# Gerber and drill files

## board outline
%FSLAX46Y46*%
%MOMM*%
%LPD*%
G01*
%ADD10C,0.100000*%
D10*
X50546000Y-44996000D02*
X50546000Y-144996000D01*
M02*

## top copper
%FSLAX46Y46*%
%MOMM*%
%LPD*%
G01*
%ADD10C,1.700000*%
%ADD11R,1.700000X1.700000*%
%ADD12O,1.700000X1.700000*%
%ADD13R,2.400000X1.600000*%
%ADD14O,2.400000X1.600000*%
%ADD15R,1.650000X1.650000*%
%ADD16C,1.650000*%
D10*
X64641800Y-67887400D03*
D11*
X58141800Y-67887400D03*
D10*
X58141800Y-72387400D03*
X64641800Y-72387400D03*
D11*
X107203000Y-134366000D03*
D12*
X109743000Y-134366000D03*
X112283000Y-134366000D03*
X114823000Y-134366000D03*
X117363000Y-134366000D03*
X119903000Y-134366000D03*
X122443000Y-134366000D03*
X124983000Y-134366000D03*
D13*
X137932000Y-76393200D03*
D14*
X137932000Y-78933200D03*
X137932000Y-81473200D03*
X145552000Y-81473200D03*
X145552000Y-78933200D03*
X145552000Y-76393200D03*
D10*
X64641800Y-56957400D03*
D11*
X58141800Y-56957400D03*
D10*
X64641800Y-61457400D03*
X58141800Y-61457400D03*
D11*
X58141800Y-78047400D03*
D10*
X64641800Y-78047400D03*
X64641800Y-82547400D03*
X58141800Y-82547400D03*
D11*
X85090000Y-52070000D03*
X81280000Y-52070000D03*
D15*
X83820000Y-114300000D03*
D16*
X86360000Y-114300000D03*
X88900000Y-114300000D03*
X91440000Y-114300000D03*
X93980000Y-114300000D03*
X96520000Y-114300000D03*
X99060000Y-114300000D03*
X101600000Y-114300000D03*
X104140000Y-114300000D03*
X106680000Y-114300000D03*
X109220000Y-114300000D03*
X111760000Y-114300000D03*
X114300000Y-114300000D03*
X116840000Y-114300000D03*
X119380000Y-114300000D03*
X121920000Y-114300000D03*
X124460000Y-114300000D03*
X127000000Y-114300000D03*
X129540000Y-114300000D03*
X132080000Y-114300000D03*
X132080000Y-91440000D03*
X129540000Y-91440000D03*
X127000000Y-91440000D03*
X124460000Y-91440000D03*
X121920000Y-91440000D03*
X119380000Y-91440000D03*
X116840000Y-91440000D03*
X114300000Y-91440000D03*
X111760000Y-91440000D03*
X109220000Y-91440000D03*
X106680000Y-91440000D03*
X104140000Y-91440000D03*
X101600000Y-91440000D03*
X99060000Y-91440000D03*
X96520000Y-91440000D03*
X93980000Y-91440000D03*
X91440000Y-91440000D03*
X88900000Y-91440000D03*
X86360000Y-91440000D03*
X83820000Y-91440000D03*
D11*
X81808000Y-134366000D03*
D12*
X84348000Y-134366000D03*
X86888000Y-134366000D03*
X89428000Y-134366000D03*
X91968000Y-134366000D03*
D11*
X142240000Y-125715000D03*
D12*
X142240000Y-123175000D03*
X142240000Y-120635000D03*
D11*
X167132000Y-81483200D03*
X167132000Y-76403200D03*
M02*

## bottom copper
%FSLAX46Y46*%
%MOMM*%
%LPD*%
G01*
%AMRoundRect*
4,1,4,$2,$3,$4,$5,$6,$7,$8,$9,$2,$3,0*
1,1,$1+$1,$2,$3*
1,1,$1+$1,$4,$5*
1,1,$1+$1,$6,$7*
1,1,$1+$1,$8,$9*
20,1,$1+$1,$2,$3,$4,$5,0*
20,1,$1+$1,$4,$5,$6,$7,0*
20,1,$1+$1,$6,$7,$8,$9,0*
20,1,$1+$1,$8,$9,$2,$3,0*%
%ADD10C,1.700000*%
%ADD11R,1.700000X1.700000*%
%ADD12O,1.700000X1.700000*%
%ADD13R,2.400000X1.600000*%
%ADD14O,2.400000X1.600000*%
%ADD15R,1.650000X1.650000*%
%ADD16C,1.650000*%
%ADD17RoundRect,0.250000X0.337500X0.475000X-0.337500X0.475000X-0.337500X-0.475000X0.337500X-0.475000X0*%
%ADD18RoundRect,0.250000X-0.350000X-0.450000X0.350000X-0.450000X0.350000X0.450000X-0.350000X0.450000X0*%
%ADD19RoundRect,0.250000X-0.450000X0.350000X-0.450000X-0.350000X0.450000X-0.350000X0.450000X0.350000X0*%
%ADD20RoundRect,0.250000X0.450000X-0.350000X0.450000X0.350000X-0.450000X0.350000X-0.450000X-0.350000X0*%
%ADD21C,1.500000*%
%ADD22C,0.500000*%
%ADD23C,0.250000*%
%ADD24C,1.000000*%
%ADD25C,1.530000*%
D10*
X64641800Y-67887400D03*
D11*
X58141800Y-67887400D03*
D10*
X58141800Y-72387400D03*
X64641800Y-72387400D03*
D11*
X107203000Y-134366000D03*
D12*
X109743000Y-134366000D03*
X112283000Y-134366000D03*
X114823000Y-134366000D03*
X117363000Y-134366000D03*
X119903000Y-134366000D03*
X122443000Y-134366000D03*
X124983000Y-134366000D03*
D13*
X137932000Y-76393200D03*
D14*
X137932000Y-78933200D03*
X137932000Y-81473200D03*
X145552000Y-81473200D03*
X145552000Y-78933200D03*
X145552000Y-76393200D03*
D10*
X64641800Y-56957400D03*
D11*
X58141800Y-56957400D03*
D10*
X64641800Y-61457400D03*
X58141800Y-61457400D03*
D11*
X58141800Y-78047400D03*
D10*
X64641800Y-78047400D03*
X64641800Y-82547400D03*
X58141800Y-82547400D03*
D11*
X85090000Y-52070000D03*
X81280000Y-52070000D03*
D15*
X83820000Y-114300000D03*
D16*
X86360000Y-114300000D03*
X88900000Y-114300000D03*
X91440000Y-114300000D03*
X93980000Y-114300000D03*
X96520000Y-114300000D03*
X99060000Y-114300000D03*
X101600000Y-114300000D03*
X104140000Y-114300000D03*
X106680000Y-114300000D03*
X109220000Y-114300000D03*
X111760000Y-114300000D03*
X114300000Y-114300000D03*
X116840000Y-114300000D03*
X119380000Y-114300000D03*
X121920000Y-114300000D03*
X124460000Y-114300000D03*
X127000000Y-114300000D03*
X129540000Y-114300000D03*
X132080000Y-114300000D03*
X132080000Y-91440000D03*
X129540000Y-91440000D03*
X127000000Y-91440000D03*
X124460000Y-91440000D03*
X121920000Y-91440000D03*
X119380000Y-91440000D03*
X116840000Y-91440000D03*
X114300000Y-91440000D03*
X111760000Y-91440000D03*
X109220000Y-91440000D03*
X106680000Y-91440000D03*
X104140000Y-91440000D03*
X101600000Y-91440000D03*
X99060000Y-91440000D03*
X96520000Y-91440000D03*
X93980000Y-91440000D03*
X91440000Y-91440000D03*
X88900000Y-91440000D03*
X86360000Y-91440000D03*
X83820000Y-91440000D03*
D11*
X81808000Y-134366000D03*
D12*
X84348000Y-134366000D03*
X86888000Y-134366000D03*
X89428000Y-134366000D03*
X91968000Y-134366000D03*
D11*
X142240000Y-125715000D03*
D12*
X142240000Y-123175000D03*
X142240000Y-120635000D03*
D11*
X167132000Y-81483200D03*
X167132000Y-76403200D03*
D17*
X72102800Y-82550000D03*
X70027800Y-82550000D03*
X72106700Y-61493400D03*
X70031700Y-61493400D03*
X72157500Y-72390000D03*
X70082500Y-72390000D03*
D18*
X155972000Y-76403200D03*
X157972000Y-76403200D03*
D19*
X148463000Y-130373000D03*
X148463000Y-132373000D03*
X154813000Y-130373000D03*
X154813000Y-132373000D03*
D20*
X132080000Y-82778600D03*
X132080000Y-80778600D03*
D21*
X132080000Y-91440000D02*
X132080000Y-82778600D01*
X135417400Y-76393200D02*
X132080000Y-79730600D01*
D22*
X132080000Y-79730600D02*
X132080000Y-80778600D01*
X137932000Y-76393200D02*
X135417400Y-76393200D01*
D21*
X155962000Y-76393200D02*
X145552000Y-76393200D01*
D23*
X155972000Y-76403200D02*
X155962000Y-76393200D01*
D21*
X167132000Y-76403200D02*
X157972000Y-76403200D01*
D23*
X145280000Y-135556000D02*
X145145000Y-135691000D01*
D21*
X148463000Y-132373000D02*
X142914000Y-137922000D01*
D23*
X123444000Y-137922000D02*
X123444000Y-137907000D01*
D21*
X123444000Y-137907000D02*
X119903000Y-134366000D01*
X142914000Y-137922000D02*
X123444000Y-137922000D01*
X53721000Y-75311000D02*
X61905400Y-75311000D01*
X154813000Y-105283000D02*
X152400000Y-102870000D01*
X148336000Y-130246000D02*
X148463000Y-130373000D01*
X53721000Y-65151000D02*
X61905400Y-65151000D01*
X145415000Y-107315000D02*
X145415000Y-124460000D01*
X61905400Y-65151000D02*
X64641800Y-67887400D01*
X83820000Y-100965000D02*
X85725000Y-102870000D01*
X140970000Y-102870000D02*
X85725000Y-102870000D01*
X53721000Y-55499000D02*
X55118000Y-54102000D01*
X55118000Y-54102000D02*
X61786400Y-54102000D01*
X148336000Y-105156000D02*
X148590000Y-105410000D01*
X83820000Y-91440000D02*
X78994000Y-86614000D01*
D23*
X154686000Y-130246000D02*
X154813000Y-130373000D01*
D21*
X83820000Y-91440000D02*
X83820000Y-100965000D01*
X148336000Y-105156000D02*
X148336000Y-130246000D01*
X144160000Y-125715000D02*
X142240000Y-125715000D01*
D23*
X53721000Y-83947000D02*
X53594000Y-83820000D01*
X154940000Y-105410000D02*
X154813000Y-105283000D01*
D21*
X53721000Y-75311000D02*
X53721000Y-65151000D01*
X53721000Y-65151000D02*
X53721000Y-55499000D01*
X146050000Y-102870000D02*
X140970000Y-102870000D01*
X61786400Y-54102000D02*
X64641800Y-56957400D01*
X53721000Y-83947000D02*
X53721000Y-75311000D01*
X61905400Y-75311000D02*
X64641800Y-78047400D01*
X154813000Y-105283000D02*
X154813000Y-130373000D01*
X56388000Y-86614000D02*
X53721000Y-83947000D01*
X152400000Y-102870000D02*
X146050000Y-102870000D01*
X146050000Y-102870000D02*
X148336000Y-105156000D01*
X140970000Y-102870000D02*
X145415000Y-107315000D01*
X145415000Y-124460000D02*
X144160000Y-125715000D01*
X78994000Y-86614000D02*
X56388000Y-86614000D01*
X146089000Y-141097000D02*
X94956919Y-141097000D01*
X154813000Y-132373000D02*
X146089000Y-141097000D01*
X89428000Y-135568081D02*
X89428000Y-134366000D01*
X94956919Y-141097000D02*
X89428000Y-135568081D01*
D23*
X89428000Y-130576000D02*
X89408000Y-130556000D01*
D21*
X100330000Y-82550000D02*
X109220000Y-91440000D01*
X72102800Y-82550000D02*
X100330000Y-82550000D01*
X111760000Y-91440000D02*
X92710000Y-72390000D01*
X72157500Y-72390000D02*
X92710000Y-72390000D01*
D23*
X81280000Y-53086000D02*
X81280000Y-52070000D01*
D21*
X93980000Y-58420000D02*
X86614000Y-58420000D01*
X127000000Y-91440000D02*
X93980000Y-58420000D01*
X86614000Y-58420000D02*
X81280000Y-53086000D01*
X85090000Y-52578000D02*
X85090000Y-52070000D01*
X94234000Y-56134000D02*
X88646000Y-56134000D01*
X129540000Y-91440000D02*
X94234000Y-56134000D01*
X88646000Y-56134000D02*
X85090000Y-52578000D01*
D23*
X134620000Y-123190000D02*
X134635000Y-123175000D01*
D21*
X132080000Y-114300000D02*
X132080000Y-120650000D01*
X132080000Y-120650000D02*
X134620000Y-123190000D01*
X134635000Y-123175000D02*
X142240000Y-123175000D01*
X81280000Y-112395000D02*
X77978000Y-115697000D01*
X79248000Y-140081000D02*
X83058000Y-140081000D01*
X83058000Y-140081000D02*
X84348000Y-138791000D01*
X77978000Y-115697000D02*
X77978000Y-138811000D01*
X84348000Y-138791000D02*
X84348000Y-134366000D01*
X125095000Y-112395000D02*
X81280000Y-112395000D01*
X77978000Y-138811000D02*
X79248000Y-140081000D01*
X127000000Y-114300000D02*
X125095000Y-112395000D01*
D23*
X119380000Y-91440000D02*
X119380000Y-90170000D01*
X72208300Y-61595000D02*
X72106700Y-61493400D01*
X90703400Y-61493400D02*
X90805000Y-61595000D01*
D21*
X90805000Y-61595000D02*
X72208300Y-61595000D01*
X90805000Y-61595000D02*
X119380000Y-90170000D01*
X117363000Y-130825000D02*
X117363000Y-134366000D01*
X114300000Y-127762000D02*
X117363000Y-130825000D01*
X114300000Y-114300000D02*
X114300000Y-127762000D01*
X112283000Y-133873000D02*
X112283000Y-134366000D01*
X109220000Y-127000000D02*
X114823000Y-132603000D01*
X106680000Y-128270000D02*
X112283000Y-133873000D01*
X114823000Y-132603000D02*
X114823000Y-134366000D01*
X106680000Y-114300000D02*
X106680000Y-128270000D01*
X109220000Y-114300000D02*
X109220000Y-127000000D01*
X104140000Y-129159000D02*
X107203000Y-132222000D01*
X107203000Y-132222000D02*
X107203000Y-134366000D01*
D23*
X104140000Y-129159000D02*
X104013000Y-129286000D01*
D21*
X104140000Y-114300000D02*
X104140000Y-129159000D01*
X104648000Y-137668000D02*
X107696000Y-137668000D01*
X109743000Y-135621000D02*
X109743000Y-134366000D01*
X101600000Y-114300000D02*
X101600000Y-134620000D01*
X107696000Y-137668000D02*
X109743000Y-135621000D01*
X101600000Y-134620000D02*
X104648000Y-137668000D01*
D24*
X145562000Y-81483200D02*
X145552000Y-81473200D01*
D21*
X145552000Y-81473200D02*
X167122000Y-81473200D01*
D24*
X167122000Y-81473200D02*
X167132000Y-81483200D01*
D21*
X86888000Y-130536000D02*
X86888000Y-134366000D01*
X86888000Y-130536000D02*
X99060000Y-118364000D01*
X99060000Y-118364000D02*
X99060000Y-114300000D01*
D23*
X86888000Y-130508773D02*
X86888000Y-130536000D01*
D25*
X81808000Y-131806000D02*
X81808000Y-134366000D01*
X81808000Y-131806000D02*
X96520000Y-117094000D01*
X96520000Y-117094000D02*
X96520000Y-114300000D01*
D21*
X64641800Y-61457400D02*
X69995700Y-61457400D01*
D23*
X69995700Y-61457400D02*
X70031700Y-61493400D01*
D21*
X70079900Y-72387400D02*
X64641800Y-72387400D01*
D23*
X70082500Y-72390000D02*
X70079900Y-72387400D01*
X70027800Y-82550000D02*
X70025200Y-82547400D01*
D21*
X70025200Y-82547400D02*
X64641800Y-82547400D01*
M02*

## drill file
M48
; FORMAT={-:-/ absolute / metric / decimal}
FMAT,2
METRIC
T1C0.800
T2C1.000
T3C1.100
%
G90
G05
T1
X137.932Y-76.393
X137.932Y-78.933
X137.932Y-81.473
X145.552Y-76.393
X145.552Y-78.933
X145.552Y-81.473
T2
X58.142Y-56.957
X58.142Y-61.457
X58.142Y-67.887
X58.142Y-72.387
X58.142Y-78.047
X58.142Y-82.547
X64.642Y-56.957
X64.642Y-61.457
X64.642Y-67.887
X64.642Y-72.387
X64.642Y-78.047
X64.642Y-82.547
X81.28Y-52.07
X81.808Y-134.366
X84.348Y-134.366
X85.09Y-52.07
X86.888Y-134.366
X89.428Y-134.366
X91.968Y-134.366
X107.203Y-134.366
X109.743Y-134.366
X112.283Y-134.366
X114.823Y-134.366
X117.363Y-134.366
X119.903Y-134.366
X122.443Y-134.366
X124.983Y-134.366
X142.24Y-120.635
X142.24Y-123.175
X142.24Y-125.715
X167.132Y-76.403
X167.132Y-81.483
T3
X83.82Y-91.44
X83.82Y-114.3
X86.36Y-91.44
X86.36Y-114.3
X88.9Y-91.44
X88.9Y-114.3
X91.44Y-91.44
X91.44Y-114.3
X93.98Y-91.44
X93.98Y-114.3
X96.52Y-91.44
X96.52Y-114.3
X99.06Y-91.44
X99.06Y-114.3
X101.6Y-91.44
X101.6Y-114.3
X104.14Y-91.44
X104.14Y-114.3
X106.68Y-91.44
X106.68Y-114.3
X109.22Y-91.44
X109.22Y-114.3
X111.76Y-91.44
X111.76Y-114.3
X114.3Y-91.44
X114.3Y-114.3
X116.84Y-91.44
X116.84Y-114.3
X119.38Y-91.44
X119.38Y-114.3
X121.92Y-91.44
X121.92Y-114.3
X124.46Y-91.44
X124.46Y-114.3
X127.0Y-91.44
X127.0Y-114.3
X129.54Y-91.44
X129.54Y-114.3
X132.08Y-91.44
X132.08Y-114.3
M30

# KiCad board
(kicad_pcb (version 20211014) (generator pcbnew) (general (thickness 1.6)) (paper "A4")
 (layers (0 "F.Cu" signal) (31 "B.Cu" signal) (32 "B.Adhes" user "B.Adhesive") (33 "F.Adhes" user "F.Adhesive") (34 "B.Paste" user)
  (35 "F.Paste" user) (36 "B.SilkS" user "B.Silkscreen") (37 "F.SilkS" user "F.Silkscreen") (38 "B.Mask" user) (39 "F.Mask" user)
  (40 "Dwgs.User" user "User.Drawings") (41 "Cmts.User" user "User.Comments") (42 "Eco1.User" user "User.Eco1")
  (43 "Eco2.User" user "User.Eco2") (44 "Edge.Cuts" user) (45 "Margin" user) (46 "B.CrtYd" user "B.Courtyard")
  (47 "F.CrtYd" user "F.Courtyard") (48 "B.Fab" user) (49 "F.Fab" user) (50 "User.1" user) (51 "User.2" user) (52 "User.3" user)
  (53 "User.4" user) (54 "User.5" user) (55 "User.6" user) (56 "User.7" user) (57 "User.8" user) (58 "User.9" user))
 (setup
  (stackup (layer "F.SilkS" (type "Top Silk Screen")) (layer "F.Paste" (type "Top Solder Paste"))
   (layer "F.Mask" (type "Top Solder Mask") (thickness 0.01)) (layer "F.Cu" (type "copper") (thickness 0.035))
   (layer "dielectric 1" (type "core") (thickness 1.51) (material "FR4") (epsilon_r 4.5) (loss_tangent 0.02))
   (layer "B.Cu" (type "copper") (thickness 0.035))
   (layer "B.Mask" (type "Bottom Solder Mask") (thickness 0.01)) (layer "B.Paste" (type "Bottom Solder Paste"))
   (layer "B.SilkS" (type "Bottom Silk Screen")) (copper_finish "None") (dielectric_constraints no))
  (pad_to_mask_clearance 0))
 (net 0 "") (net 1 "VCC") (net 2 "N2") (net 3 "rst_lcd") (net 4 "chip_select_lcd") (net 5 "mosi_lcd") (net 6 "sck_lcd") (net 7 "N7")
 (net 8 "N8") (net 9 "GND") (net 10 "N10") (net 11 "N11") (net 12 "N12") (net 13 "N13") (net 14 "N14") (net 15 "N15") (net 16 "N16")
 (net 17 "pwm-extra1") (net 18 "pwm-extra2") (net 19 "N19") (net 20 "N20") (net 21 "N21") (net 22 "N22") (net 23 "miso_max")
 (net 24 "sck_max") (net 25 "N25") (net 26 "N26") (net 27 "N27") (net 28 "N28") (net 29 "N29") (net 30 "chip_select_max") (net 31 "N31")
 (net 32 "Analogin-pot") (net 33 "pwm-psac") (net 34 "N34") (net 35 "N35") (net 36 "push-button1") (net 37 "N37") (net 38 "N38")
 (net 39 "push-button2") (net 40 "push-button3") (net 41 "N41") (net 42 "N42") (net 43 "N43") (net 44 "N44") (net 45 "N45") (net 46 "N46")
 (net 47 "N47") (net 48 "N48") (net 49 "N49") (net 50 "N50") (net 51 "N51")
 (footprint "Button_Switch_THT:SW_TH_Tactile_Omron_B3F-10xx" (layer "F.Cu") (at 58.1418 67.8874)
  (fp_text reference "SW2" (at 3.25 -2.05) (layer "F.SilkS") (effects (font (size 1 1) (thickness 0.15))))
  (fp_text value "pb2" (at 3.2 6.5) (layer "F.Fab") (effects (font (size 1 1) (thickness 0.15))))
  (pad "1" thru_hole circle (at 6.5 0) (size 1.7 1.7) (drill 1) (layers *.Cu *.Mask) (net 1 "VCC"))
  (pad "1" thru_hole rect (at 0 0) (size 1.7 1.7) (drill 1) (layers *.Cu *.Mask) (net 1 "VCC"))
  (pad "2" thru_hole circle (at 0 4.5) (size 1.7 1.7) (drill 1) (layers *.Cu *.Mask) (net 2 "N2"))
  (pad "2" thru_hole circle (at 6.5 4.5) (size 1.7 1.7) (drill 1) (layers *.Cu *.Mask) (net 2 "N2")))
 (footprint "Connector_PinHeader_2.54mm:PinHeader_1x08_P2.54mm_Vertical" (layer "F.Cu") (at 107.203 134.366 90)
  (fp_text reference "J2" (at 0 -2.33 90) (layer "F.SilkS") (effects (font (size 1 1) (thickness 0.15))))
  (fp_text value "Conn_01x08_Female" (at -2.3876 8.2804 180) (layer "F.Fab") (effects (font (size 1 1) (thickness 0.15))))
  (pad "1" thru_hole rect (at 0 0 90) (size 1.7 1.7) (drill 1) (layers *.Cu *.Mask) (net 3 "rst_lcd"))
  (pad "2" thru_hole oval (at 0 2.54 90) (size 1.7 1.7) (drill 1) (layers *.Cu *.Mask) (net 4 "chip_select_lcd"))
  (pad "3" thru_hole oval (at 0 5.08 90) (size 1.7 1.7) (drill 1) (layers *.Cu *.Mask) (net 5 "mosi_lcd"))
  (pad "4" thru_hole oval (at 0 7.62 90) (size 1.7 1.7) (drill 1) (layers *.Cu *.Mask) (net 5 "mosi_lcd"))
  (pad "5" thru_hole oval (at 0 10.16 90) (size 1.7 1.7) (drill 1) (layers *.Cu *.Mask) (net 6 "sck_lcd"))
  (pad "6" thru_hole oval (at 0 12.7 90) (size 1.7 1.7) (drill 1) (layers *.Cu *.Mask) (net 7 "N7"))
  (pad "7" thru_hole oval (at 0 15.24 90) (size 1.7 1.7) (drill 1) (layers *.Cu *.Mask) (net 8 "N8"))
  (pad "8" thru_hole oval (at 0 17.78 90) (size 1.7 1.7) (drill 1) (layers *.Cu *.Mask) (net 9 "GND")))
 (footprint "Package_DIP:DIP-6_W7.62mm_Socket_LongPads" (layer "F.Cu") (at 137.932 76.3932)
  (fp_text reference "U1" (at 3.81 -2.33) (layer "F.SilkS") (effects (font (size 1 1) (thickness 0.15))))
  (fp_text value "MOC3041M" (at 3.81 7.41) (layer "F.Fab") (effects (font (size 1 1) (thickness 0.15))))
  (pad "1" thru_hole rect (at 0 0) (size 2.4 1.6) (drill 0.8) (layers *.Cu *.Mask) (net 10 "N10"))
  (pad "2" thru_hole oval (at 0 2.54) (size 2.4 1.6) (drill 0.8) (layers *.Cu *.Mask) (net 9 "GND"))
  (pad "3" thru_hole oval (at 0 5.08) (size 2.4 1.6) (drill 0.8) (layers *.Cu *.Mask) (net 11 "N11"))
  (pad "4" thru_hole oval (at 7.62 5.08) (size 2.4 1.6) (drill 0.8) (layers *.Cu *.Mask) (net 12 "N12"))
  (pad "5" thru_hole oval (at 7.62 2.54) (size 2.4 1.6) (drill 0.8) (layers *.Cu *.Mask) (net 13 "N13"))
  (pad "6" thru_hole oval (at 7.62 0) (size 2.4 1.6) (drill 0.8) (layers *.Cu *.Mask) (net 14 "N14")))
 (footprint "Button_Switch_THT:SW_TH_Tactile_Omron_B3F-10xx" (layer "F.Cu") (at 58.1418 56.9574)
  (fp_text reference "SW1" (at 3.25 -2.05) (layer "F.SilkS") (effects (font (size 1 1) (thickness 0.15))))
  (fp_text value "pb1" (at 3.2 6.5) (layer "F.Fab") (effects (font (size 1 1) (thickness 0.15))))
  (pad "1" thru_hole circle (at 6.5 0) (size 1.7 1.7) (drill 1) (layers *.Cu *.Mask) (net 1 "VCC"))
  (pad "1" thru_hole rect (at 0 0) (size 1.7 1.7) (drill 1) (layers *.Cu *.Mask) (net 1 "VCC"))
  (pad "2" thru_hole circle (at 6.5 4.5) (size 1.7 1.7) (drill 1) (layers *.Cu *.Mask) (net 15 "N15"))
  (pad "2" thru_hole circle (at 0 4.5) (size 1.7 1.7) (drill 1) (layers *.Cu *.Mask) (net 15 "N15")))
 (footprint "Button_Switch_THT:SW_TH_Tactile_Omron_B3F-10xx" (layer "F.Cu") (at 58.1418 78.0474)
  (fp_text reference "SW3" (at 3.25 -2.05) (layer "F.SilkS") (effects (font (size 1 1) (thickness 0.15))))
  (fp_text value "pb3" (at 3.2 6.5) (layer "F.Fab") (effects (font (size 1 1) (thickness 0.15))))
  (pad "1" thru_hole rect (at 0 0) (size 1.7 1.7) (drill 1) (layers *.Cu *.Mask) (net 1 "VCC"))
  (pad "1" thru_hole circle (at 6.5 0) (size 1.7 1.7) (drill 1) (layers *.Cu *.Mask) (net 1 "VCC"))
  (pad "2" thru_hole circle (at 6.5 4.5) (size 1.7 1.7) (drill 1) (layers *.Cu *.Mask) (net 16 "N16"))
  (pad "2" thru_hole circle (at 0 4.5) (size 1.7 1.7) (drill 1) (layers *.Cu *.Mask) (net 16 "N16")))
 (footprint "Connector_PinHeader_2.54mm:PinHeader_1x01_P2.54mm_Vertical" (layer "F.Cu") (at 85.09 52.07)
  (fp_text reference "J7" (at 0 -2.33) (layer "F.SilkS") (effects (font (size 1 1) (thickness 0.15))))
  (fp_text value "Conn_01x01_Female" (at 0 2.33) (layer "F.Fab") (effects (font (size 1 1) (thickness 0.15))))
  (pad "1" thru_hole rect (at 0 0) (size 1.7 1.7) (drill 1) (layers *.Cu *.Mask) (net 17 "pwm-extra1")))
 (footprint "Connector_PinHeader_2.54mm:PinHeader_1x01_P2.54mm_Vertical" (layer "F.Cu") (at 81.28 52.07)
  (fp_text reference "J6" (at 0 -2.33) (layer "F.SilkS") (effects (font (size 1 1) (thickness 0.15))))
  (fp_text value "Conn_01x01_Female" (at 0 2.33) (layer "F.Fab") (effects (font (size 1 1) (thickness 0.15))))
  (pad "1" thru_hole rect (at 0 0) (size 1.7 1.7) (drill 1) (layers *.Cu *.Mask) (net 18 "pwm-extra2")))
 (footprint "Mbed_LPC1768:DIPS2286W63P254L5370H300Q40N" (layer "F.Cu") (at 83.82 114.3 90)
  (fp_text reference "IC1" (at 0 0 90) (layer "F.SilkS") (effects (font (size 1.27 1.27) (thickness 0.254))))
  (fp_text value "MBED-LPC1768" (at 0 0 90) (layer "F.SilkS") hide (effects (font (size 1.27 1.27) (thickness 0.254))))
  (pad "1" thru_hole rect locked (at 0 0 90) (size 1.65 1.65) (drill 1.1) (layers *.Cu *.Mask) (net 9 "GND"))
  (pad "2" thru_hole circle locked (at 0 2.54 90) (size 1.65 1.65) (drill 1.1) (layers *.Cu *.Mask) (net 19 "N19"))
  (pad "3" thru_hole circle locked (at 0 5.08 90) (size 1.65 1.65) (drill 1.1) (layers *.Cu *.Mask) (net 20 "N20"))
  (pad "4" thru_hole circle locked (at 0 7.62 90) (size 1.65 1.65) (drill 1.1) (layers *.Cu *.Mask) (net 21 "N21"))
  (pad "5" thru_hole circle locked (at 0 10.16 90) (size 1.65 1.65) (drill 1.1) (layers *.Cu *.Mask) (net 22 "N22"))
  (pad "6" thru_hole circle locked (at 0 12.7 90) (size 1.65 1.65) (drill 1.1) (layers *.Cu *.Mask) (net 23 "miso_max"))
  (pad "7" thru_hole circle locked (at 0 15.24 90) (size 1.65 1.65) (drill 1.1) (layers *.Cu *.Mask) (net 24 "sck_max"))
  (pad "8" thru_hole circle locked (at 0 17.78 90) (size 1.65 1.65) (drill 1.1) (layers *.Cu *.Mask) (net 4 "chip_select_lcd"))
  (pad "9" thru_hole circle locked (at 0 20.32 90) (size 1.65 1.65) (drill 1.1) (layers *.Cu *.Mask) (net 3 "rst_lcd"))
  (pad "10" thru_hole circle locked (at 0 22.86 90) (size 1.65 1.65) (drill 1.1) (layers *.Cu *.Mask) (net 5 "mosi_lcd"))
  (pad "11" thru_hole circle locked (at 0 25.4 90) (size 1.65 1.65) (drill 1.1) (layers *.Cu *.Mask) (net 5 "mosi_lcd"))
  (pad "12" thru_hole circle locked (at 0 27.94 90) (size 1.65 1.65) (drill 1.1) (layers *.Cu *.Mask) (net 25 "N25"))
  (pad "13" thru_hole circle locked (at 0 30.48 90) (size 1.65 1.65) (drill 1.1) (layers *.Cu *.Mask) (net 6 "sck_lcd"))
  (pad "14" thru_hole circle locked (at 0 33.02 90) (size 1.65 1.65) (drill 1.1) (layers *.Cu *.Mask) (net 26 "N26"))
  (pad "15" thru_hole circle locked (at 0 35.56 90) (size 1.65 1.65) (drill 1.1) (layers *.Cu *.Mask) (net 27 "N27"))
  (pad "16" thru_hole circle locked (at 0 38.1 90) (size 1.65 1.65) (drill 1.1) (layers *.Cu *.Mask) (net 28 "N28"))
  (pad "17" thru_hole circle locked (at 0 40.64 90) (size 1.65 1.65) (drill 1.1) (layers *.Cu *.Mask) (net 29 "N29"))
  (pad "18" thru_hole circle locked (at 0 43.18 90) (size 1.65 1.65) (drill 1.1) (layers *.Cu *.Mask) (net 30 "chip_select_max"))
  (pad "19" thru_hole circle locked (at 0 45.72 90) (size 1.65 1.65) (drill 1.1) (layers *.Cu *.Mask) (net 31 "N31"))
  (pad "20" thru_hole circle locked (at 0 48.26 90) (size 1.65 1.65) (drill 1.1) (layers *.Cu *.Mask) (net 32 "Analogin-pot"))
  (pad "21" thru_hole circle locked (at 22.86 48.26 90) (size 1.65 1.65) (drill 1.1) (layers *.Cu *.Mask) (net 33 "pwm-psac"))
  (pad "22" thru_hole circle locked (at 22.86 45.72 90) (size 1.65 1.65) (drill 1.1) (layers *.Cu *.Mask) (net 17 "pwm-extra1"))
  (pad "23" thru_hole circle locked (at 22.86 43.18 90) (size 1.65 1.65) (drill 1.1) (layers *.Cu *.Mask) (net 18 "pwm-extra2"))
  (pad "24" thru_hole circle locked (at 22.86 40.64 90) (size 1.65 1.65) (drill 1.1) (layers *.Cu *.Mask) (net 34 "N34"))
  (pad "25" thru_hole circle locked (at 22.86 38.1 90) (size 1.65 1.65) (drill 1.1) (layers *.Cu *.Mask) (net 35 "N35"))
  (pad "26" thru_hole circle locked (at 22.86 35.56 90) (size 1.65 1.65) (drill 1.1) (layers *.Cu *.Mask) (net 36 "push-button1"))
  (pad "27" thru_hole circle locked (at 22.86 33.02 90) (size 1.65 1.65) (drill 1.1) (layers *.Cu *.Mask) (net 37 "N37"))
  (pad "28" thru_hole circle locked (at 22.86 30.48 90) (size 1.65 1.65) (drill 1.1) (layers *.Cu *.Mask) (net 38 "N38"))
  (pad "29" thru_hole circle locked (at 22.86 27.94 90) (size 1.65 1.65) (drill 1.1) (layers *.Cu *.Mask) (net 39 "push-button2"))
  (pad "30" thru_hole circle locked (at 22.86 25.4 90) (size 1.65 1.65) (drill 1.1) (layers *.Cu *.Mask) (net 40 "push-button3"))
  (pad "31" thru_hole circle locked (at 22.86 22.86 90) (size 1.65 1.65) (drill 1.1) (layers *.Cu *.Mask) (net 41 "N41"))
  (pad "32" thru_hole circle locked (at 22.86 20.32 90) (size 1.65 1.65) (drill 1.1) (layers *.Cu *.Mask) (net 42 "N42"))
  (pad "33" thru_hole circle locked (at 22.86 17.78 90) (size 1.65 1.65) (drill 1.1) (layers *.Cu *.Mask) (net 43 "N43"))
  (pad "34" thru_hole circle locked (at 22.86 15.24 90) (size 1.65 1.65) (drill 1.1) (layers *.Cu *.Mask) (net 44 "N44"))
  (pad "35" thru_hole circle locked (at 22.86 12.7 90) (size 1.65 1.65) (drill 1.1) (layers *.Cu *.Mask) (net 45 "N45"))
  (pad "36" thru_hole circle locked (at 22.86 10.16 90) (size 1.65 1.65) (drill 1.1) (layers *.Cu *.Mask) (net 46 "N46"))
  (pad "37" thru_hole circle locked (at 22.86 7.62 90) (size 1.65 1.65) (drill 1.1) (layers *.Cu *.Mask) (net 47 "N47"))
  (pad "38" thru_hole circle locked (at 22.86 5.08 90) (size 1.65 1.65) (drill 1.1) (layers *.Cu *.Mask) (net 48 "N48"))
  (pad "39" thru_hole circle locked (at 22.86 2.54 90) (size 1.65 1.65) (drill 1.1) (layers *.Cu *.Mask) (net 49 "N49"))
  (pad "40" thru_hole circle locked (at 22.86 0 90) (size 1.65 1.65) (drill 1.1) (layers *.Cu *.Mask) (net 1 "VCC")))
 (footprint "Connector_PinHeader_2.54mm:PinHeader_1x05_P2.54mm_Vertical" (layer "F.Cu") (at 81.808 134.366 90)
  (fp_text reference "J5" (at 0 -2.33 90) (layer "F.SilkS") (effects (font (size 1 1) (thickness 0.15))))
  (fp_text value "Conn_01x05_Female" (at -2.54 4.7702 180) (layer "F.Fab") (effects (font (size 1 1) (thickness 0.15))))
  (pad "1" thru_hole rect (at 0 0 90) (size 1.7 1.7) (drill 1) (layers *.Cu *.Mask) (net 23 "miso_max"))
  (pad "2" thru_hole oval (at 0 2.54 90) (size 1.7 1.7) (drill 1) (layers *.Cu *.Mask) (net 30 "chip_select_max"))
  (pad "3" thru_hole oval (at 0 5.08 90) (size 1.7 1.7) (drill 1) (layers *.Cu *.Mask) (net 24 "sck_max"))
  (pad "4" thru_hole oval (at 0 7.62 90) (size 1.7 1.7) (drill 1) (layers *.Cu *.Mask) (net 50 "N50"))
  (pad "5" thru_hole oval (at 0 10.16 90) (size 1.7 1.7) (drill 1) (layers *.Cu *.Mask) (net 9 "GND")))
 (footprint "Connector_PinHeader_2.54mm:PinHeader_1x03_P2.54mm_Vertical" (layer "F.Cu") (at 142.24 125.715 180)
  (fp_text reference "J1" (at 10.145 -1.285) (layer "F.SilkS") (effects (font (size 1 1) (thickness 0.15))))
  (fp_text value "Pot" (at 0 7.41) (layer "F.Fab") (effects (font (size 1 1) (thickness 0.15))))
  (pad "1" thru_hole rect (at 0 0 180) (size 1.7 1.7) (drill 1) (layers *.Cu *.Mask) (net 1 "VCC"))
  (pad "2" thru_hole oval (at 0 2.54 180) (size 1.7 1.7) (drill 1) (layers *.Cu *.Mask) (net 32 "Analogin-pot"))
  (pad "3" thru_hole oval (at 0 5.08 180) (size 1.7 1.7) (drill 1) (layers *.Cu *.Mask) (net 9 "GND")))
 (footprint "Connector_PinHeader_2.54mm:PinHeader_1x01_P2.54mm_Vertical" (layer "F.Cu") (at 167.132 81.4832)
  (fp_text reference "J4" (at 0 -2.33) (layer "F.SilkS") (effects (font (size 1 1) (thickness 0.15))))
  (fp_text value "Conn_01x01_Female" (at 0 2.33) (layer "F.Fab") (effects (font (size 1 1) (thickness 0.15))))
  (pad "1" thru_hole rect (at 0 0) (size 1.7 1.7) (drill 1) (layers *.Cu *.Mask) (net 12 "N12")))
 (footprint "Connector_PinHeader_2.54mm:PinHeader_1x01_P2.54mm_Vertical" (layer "F.Cu") (at 167.132 76.4032)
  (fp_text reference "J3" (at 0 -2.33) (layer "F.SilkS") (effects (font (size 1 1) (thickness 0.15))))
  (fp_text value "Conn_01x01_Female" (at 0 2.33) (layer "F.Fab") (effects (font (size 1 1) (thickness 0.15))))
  (pad "1" thru_hole rect (at 0 0) (size 1.7 1.7) (drill 1) (layers *.Cu *.Mask) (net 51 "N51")))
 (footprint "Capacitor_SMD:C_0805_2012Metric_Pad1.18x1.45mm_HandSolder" (layer "B.Cu") (at 71.0653 82.55 180)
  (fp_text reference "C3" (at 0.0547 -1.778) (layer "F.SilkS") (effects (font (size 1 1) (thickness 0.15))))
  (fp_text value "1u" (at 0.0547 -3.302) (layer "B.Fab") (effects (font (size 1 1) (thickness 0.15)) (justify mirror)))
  (pad "1" smd roundrect (at -1.0375 0 180) (size 1.175 1.45) (layers "B.Cu" "B.Paste" "B.Mask") (roundrect_rratio 0.212766)
   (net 40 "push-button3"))
  (pad "2" smd roundrect (at 1.0375 0 180) (size 1.175 1.45) (layers "B.Cu" "B.Paste" "B.Mask") (roundrect_rratio 0.212766) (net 16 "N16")))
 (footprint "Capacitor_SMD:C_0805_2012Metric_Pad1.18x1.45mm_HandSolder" (layer "B.Cu") (at 71.0692 61.4934 180)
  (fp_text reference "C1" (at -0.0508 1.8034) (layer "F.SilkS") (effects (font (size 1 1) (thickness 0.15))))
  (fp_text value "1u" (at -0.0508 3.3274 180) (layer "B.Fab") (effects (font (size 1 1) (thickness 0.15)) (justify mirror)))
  (pad "1" smd roundrect (at -1.0375 0 180) (size 1.175 1.45) (layers "B.Cu" "B.Paste" "B.Mask") (roundrect_rratio 0.212766)
   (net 36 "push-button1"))
  (pad "2" smd roundrect (at 1.0375 0 180) (size 1.175 1.45) (layers "B.Cu" "B.Paste" "B.Mask") (roundrect_rratio 0.212766) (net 15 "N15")))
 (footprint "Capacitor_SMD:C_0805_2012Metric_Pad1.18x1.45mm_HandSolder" (layer "B.Cu") (at 71.12 72.39 180)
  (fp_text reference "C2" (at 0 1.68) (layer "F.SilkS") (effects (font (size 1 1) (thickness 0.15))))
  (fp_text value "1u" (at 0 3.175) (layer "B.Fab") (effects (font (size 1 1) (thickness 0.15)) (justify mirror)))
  (pad "1" smd roundrect (at -1.0375 0 180) (size 1.175 1.45) (layers "B.Cu" "B.Paste" "B.Mask") (roundrect_rratio 0.212766)
   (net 39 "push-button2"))
  (pad "2" smd roundrect (at 1.0375 0 180) (size 1.175 1.45) (layers "B.Cu" "B.Paste" "B.Mask") (roundrect_rratio 0.212766) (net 2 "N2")))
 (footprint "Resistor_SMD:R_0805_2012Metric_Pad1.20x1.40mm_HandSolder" (layer "B.Cu") (at 156.972 76.4032)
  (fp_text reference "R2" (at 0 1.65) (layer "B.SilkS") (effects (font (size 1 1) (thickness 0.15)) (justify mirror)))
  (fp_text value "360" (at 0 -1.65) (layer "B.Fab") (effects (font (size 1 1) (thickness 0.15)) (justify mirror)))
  (pad "1" smd roundrect (at -1 0) (size 1.2 1.4) (layers "B.Cu" "B.Paste" "B.Mask") (roundrect_rratio 0.2083333333) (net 14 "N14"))
  (pad "2" smd roundrect (at 1 0) (size 1.2 1.4) (layers "B.Cu" "B.Paste" "B.Mask") (roundrect_rratio 0.2083333333) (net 51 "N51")))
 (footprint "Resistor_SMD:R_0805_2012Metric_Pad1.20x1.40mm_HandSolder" (layer "B.Cu") (at 148.463 131.373 -90)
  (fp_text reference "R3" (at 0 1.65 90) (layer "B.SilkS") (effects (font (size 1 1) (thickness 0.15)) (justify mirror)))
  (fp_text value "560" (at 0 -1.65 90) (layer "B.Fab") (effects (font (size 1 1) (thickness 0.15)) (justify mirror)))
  (pad "1" smd roundrect (at -1 0 270) (size 1.2 1.4) (layers "B.Cu" "B.Paste" "B.Mask") (roundrect_rratio 0.208333) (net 1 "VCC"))
  (pad "2" smd roundrect (at 1 0 270) (size 1.2 1.4) (layers "B.Cu" "B.Paste" "B.Mask") (roundrect_rratio 0.208333) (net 7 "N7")))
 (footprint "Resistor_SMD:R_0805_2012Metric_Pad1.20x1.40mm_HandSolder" (layer "B.Cu") (at 154.813 131.373 -90)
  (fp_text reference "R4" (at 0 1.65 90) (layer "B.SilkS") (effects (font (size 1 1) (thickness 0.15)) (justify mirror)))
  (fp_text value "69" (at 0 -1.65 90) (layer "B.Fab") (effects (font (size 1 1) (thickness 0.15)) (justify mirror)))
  (pad "1" smd roundrect (at -1 0 270) (size 1.2 1.4) (layers "B.Cu" "B.Paste" "B.Mask") (roundrect_rratio 0.208333) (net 1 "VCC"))
  (pad "2" smd roundrect (at 1 0 270) (size 1.2 1.4) (layers "B.Cu" "B.Paste" "B.Mask") (roundrect_rratio 0.208333) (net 50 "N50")))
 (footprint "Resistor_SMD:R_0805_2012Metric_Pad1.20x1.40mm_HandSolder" (layer "B.Cu") (at 132.08 81.7786 90)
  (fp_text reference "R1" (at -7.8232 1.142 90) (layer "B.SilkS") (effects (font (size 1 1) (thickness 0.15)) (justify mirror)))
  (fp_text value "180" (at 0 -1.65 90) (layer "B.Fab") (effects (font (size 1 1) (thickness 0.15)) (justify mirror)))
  (pad "1" smd roundrect (at -1 0 90) (size 1.2 1.4) (layers "B.Cu" "B.Paste" "B.Mask") (roundrect_rratio 0.2083333333) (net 33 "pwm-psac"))
  (pad "2" smd roundrect (at 1 0 90) (size 1.2 1.4) (layers "B.Cu" "B.Paste" "B.Mask") (roundrect_rratio 0.2083333333) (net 10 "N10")))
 (gr_line (start 50.546 44.996) (end 50.546 144.996) (layer "Edge.Cuts") (width 0.1))
 (segment (start 132.08 91.44) (end 132.08 82.7786) (width 1.5) (layer "B.Cu") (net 33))
 (segment (start 135.4174 76.3932) (end 132.08 79.7306) (width 1.5) (layer "B.Cu") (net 10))
 (segment (start 132.08 79.7306) (end 132.08 80.7786) (width 0.5) (layer "B.Cu") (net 10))
 (segment (start 137.932 76.3932) (end 135.4174 76.3932) (width 0.5) (layer "B.Cu") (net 10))
 (segment (start 155.962 76.3932) (end 145.552 76.3932) (width 1.5) (layer "B.Cu") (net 14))
 (segment (start 155.972 76.4032) (end 155.962 76.3932) (width 0.25) (layer "B.Cu") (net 14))
 (segment (start 167.132 76.4032) (end 157.972 76.4032) (width 1.5) (layer "B.Cu") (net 51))
 (segment (start 145.28 135.556) (end 145.145 135.691) (width 0.25) (layer "B.Cu") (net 7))
 (segment (start 148.463 132.373) (end 142.914 137.922) (width 1.5) (layer "B.Cu") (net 7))
 (segment (start 123.444 137.922) (end 123.444 137.907) (width 0.25) (layer "B.Cu") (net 7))
 (segment (start 123.444 137.907) (end 119.903 134.366) (width 1.5) (layer "B.Cu") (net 7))
 (segment (start 142.914 137.922) (end 123.444 137.922) (width 1.5) (layer "B.Cu") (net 7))
 (segment (start 53.721 75.311) (end 61.9054 75.311) (width 1.5) (layer "B.Cu") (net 1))
 (segment (start 154.813 105.283) (end 152.4 102.87) (width 1.5) (layer "B.Cu") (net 1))
 (segment (start 148.336 130.246) (end 148.463 130.373) (width 1.5) (layer "B.Cu") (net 1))
 (segment (start 53.721 65.151) (end 61.9054 65.151) (width 1.5) (layer "B.Cu") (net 1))
 (segment (start 145.415 107.315) (end 145.415 124.46) (width 1.5) (layer "B.Cu") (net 1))
 (segment (start 61.9054 65.151) (end 64.6418 67.8874) (width 1.5) (layer "B.Cu") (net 1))
 (segment (start 83.82 100.965) (end 85.725 102.87) (width 1.5) (layer "B.Cu") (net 1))
 (segment (start 140.97 102.87) (end 85.725 102.87) (width 1.5) (layer "B.Cu") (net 1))
 (segment (start 53.721 55.499) (end 55.118 54.102) (width 1.5) (layer "B.Cu") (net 1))
 (segment (start 55.118 54.102) (end 61.7864 54.102) (width 1.5) (layer "B.Cu") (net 1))
 (segment (start 148.336 105.156) (end 148.59 105.41) (width 1.5) (layer "B.Cu") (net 1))
 (segment (start 83.82 91.44) (end 78.994 86.614) (width 1.5) (layer "B.Cu") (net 1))
 (segment (start 154.686 130.246) (end 154.813 130.373) (width 0.25) (layer "B.Cu") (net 1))
 (segment (start 83.82 91.44) (end 83.82 100.965) (width 1.5) (layer "B.Cu") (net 1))
 (segment (start 148.336 105.156) (end 148.336 130.246) (width 1.5) (layer "B.Cu") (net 1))
 (segment (start 144.16 125.715) (end 142.24 125.715) (width 1.5) (layer "B.Cu") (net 1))
 (segment (start 53.721 83.947) (end 53.594 83.82) (width 0.25) (layer "B.Cu") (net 1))
 (segment (start 154.94 105.41) (end 154.813 105.283) (width 0.25) (layer "B.Cu") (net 1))
 (segment (start 53.721 75.311) (end 53.721 65.151) (width 1.5) (layer "B.Cu") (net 1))
 (segment (start 53.721 65.151) (end 53.721 55.499) (width 1.5) (layer "B.Cu") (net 1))
 (segment (start 146.05 102.87) (end 140.97 102.87) (width 1.5) (layer "B.Cu") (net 1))
 (segment (start 61.7864 54.102) (end 64.6418 56.9574) (width 1.5) (layer "B.Cu") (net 1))
 (segment (start 53.721 83.947) (end 53.721 75.311) (width 1.5) (layer "B.Cu") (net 1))
 (segment (start 61.9054 75.311) (end 64.6418 78.0474) (width 1.5) (layer "B.Cu") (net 1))
 (segment (start 154.813 105.283) (end 154.813 130.373) (width 1.5) (layer "B.Cu") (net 1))
 (segment (start 56.388 86.614) (end 53.721 83.947) (width 1.5) (layer "B.Cu") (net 1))
 (segment (start 152.4 102.87) (end 146.05 102.87) (width 1.5) (layer "B.Cu") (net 1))
 (segment (start 146.05 102.87) (end 148.336 105.156) (width 1.5) (layer "B.Cu") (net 1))
 (segment (start 140.97 102.87) (end 145.415 107.315) (width 1.5) (layer "B.Cu") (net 1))
 (segment (start 145.415 124.46) (end 144.16 125.715) (width 1.5) (layer "B.Cu") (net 1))
 (segment (start 78.994 86.614) (end 56.388 86.614) (width 1.5) (layer "B.Cu") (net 1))
 (segment (start 146.089 141.097) (end 94.956919 141.097) (width 1.5) (layer "B.Cu") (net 50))
 (segment (start 154.813 132.373) (end 146.089 141.097) (width 1.5) (layer "B.Cu") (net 50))
 (segment (start 89.428 135.568081) (end 89.428 134.366) (width 1.5) (layer "B.Cu") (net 50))
 (segment (start 94.956919 141.097) (end 89.428 135.568081) (width 1.5) (layer "B.Cu") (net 50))
 (segment (start 89.428 130.576) (end 89.408 130.556) (width 0.25) (layer "B.Cu") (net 50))
 (segment (start 100.33 82.55) (end 109.22 91.44) (width 1.5) (layer "B.Cu") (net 40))
 (segment (start 72.1028 82.55) (end 100.33 82.55) (width 1.5) (layer "B.Cu") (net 40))
 (segment (start 111.76 91.44) (end 92.71 72.39) (width 1.5) (layer "B.Cu") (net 39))
 (segment (start 72.1575 72.39) (end 92.71 72.39) (width 1.5) (layer "B.Cu") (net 39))
 (segment (start 81.28 53.086) (end 81.28 52.07) (width 0.25) (layer "B.Cu") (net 18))
 (segment (start 93.98 58.42) (end 86.614 58.42) (width 1.5) (layer "B.Cu") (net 18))
 (segment (start 127 91.44) (end 93.98 58.42) (width 1.5) (layer "B.Cu") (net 18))
 (segment (start 86.614 58.42) (end 81.28 53.086) (width 1.5) (layer "B.Cu") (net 18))
 (segment (start 85.09 52.578) (end 85.09 52.07) (width 1.5) (layer "B.Cu") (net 17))
 (segment (start 94.234 56.134) (end 88.646 56.134) (width 1.5) (layer "B.Cu") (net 17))
 (segment (start 129.54 91.44) (end 94.234 56.134) (width 1.5) (layer "B.Cu") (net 17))
 (segment (start 88.646 56.134) (end 85.09 52.578) (width 1.5) (layer "B.Cu") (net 17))
 (segment (start 134.62 123.19) (end 134.635 123.175) (width 0.25) (layer "B.Cu") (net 32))
 (segment (start 132.08 114.3) (end 132.08 120.65) (width 1.5) (layer "B.Cu") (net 32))
 (segment (start 132.08 120.65) (end 134.62 123.19) (width 1.5) (layer "B.Cu") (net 32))
 (segment (start 134.635 123.175) (end 142.24 123.175) (width 1.5) (layer "B.Cu") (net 32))
 (segment (start 81.28 112.395) (end 77.978 115.697) (width 1.5) (layer "B.Cu") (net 30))
 (segment (start 79.248 140.081) (end 83.058 140.081) (width 1.5) (layer "B.Cu") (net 30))
 (segment (start 83.058 140.081) (end 84.348 138.791) (width 1.5) (layer "B.Cu") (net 30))
 (segment (start 77.978 115.697) (end 77.978 138.811) (width 1.5) (layer "B.Cu") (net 30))
 (segment (start 84.348 138.791) (end 84.348 134.366) (width 1.5) (layer "B.Cu") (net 30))
 (segment (start 125.095 112.395) (end 81.28 112.395) (width 1.5) (layer "B.Cu") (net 30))
 (segment (start 77.978 138.811) (end 79.248 140.081) (width 1.5) (layer "B.Cu") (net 30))
 (segment (start 127 114.3) (end 125.095 112.395) (width 1.5) (layer "B.Cu") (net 30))
 (segment (start 119.38 91.44) (end 119.38 90.17) (width 0.25) (layer "B.Cu") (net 36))
 (segment (start 72.2083 61.595) (end 72.1067 61.4934) (width 0.25) (layer "B.Cu") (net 36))
 (segment (start 90.7034 61.4934) (end 90.805 61.595) (width 0.25) (layer "B.Cu") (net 36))
 (segment (start 90.805 61.595) (end 72.2083 61.595) (width 1.5) (layer "B.Cu") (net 36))
 (segment (start 90.805 61.595) (end 119.38 90.17) (width 1.5) (layer "B.Cu") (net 36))
 (segment (start 117.363 130.825) (end 117.363 134.366) (width 1.5) (layer "B.Cu") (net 6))
 (segment (start 114.3 127.762) (end 117.363 130.825) (width 1.5) (layer "B.Cu") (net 6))
 (segment (start 114.3 114.3) (end 114.3 127.762) (width 1.5) (layer "B.Cu") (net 6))
 (segment (start 112.283 133.873) (end 112.283 134.366) (width 1.5) (layer "B.Cu") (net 5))
 (segment (start 109.22 127) (end 114.823 132.603) (width 1.5) (layer "B.Cu") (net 5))
 (segment (start 106.68 128.27) (end 112.283 133.873) (width 1.5) (layer "B.Cu") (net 5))
 (segment (start 114.823 132.603) (end 114.823 134.366) (width 1.5) (layer "B.Cu") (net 5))
 (segment (start 106.68 114.3) (end 106.68 128.27) (width 1.5) (layer "B.Cu") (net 5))
 (segment (start 109.22 114.3) (end 109.22 127) (width 1.5) (layer "B.Cu") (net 5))
 (segment (start 104.14 129.159) (end 107.203 132.222) (width 1.5) (layer "B.Cu") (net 3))
 (segment (start 107.203 132.222) (end 107.203 134.366) (width 1.5) (layer "B.Cu") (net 3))
 (segment (start 104.14 129.159) (end 104.013 129.286) (width 0.25) (layer "B.Cu") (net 3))
 (segment (start 104.14 114.3) (end 104.14 129.159) (width 1.5) (layer "B.Cu") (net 3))
 (segment (start 104.648 137.668) (end 107.696 137.668) (width 1.5) (layer "B.Cu") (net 4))
 (segment (start 109.743 135.621) (end 109.743 134.366) (width 1.5) (layer "B.Cu") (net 4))
 (segment (start 101.6 114.3) (end 101.6 134.62) (width 1.5) (layer "B.Cu") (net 4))
 (segment (start 107.696 137.668) (end 109.743 135.621) (width 1.5) (layer "B.Cu") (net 4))
 (segment (start 101.6 134.62) (end 104.648 137.668) (width 1.5) (layer "B.Cu") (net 4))
 (segment (start 145.562 81.4832) (end 145.552 81.4732) (width 1) (layer "B.Cu") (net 12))
 (segment (start 145.552 81.4732) (end 167.122 81.4732) (width 1.5) (layer "B.Cu") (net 12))
 (segment (start 167.122 81.4732) (end 167.132 81.4832) (width 1) (layer "B.Cu") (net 12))
 (segment (start 86.888 130.536) (end 86.888 134.366) (width 1.5) (layer "B.Cu") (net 24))
 (segment (start 86.888 130.536) (end 99.06 118.364) (width 1.5) (layer "B.Cu") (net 24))
 (segment (start 99.06 118.364) (end 99.06 114.3) (width 1.5) (layer "B.Cu") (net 24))
 (segment (start 86.888 130.508773) (end 86.888 130.536) (width 0.25) (layer "B.Cu") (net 24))
 (segment (start 81.808 131.806) (end 81.808 134.366) (width 1.53) (layer "B.Cu") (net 23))
 (segment (start 81.808 131.806) (end 96.52 117.094) (width 1.53) (layer "B.Cu") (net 23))
 (segment (start 96.52 117.094) (end 96.52 114.3) (width 1.53) (layer "B.Cu") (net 23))
 (segment (start 64.6418 61.4574) (end 69.9957 61.4574) (width 1.5) (layer "B.Cu") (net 15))
 (segment (start 69.9957 61.4574) (end 70.0317 61.4934) (width 0.25) (layer "B.Cu") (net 15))
 (segment (start 70.0799 72.3874) (end 64.6418 72.3874) (width 1.5) (layer "B.Cu") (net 2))
 (segment (start 70.0825 72.39) (end 70.0799 72.3874) (width 0.25) (layer "B.Cu") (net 2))
 (segment (start 70.0278 82.55) (end 70.0252 82.5474) (width 0.25) (layer "B.Cu") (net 16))
 (segment (start 70.0252 82.5474) (end 64.6418 82.5474) (width 1.5) (layer "B.Cu") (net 16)))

